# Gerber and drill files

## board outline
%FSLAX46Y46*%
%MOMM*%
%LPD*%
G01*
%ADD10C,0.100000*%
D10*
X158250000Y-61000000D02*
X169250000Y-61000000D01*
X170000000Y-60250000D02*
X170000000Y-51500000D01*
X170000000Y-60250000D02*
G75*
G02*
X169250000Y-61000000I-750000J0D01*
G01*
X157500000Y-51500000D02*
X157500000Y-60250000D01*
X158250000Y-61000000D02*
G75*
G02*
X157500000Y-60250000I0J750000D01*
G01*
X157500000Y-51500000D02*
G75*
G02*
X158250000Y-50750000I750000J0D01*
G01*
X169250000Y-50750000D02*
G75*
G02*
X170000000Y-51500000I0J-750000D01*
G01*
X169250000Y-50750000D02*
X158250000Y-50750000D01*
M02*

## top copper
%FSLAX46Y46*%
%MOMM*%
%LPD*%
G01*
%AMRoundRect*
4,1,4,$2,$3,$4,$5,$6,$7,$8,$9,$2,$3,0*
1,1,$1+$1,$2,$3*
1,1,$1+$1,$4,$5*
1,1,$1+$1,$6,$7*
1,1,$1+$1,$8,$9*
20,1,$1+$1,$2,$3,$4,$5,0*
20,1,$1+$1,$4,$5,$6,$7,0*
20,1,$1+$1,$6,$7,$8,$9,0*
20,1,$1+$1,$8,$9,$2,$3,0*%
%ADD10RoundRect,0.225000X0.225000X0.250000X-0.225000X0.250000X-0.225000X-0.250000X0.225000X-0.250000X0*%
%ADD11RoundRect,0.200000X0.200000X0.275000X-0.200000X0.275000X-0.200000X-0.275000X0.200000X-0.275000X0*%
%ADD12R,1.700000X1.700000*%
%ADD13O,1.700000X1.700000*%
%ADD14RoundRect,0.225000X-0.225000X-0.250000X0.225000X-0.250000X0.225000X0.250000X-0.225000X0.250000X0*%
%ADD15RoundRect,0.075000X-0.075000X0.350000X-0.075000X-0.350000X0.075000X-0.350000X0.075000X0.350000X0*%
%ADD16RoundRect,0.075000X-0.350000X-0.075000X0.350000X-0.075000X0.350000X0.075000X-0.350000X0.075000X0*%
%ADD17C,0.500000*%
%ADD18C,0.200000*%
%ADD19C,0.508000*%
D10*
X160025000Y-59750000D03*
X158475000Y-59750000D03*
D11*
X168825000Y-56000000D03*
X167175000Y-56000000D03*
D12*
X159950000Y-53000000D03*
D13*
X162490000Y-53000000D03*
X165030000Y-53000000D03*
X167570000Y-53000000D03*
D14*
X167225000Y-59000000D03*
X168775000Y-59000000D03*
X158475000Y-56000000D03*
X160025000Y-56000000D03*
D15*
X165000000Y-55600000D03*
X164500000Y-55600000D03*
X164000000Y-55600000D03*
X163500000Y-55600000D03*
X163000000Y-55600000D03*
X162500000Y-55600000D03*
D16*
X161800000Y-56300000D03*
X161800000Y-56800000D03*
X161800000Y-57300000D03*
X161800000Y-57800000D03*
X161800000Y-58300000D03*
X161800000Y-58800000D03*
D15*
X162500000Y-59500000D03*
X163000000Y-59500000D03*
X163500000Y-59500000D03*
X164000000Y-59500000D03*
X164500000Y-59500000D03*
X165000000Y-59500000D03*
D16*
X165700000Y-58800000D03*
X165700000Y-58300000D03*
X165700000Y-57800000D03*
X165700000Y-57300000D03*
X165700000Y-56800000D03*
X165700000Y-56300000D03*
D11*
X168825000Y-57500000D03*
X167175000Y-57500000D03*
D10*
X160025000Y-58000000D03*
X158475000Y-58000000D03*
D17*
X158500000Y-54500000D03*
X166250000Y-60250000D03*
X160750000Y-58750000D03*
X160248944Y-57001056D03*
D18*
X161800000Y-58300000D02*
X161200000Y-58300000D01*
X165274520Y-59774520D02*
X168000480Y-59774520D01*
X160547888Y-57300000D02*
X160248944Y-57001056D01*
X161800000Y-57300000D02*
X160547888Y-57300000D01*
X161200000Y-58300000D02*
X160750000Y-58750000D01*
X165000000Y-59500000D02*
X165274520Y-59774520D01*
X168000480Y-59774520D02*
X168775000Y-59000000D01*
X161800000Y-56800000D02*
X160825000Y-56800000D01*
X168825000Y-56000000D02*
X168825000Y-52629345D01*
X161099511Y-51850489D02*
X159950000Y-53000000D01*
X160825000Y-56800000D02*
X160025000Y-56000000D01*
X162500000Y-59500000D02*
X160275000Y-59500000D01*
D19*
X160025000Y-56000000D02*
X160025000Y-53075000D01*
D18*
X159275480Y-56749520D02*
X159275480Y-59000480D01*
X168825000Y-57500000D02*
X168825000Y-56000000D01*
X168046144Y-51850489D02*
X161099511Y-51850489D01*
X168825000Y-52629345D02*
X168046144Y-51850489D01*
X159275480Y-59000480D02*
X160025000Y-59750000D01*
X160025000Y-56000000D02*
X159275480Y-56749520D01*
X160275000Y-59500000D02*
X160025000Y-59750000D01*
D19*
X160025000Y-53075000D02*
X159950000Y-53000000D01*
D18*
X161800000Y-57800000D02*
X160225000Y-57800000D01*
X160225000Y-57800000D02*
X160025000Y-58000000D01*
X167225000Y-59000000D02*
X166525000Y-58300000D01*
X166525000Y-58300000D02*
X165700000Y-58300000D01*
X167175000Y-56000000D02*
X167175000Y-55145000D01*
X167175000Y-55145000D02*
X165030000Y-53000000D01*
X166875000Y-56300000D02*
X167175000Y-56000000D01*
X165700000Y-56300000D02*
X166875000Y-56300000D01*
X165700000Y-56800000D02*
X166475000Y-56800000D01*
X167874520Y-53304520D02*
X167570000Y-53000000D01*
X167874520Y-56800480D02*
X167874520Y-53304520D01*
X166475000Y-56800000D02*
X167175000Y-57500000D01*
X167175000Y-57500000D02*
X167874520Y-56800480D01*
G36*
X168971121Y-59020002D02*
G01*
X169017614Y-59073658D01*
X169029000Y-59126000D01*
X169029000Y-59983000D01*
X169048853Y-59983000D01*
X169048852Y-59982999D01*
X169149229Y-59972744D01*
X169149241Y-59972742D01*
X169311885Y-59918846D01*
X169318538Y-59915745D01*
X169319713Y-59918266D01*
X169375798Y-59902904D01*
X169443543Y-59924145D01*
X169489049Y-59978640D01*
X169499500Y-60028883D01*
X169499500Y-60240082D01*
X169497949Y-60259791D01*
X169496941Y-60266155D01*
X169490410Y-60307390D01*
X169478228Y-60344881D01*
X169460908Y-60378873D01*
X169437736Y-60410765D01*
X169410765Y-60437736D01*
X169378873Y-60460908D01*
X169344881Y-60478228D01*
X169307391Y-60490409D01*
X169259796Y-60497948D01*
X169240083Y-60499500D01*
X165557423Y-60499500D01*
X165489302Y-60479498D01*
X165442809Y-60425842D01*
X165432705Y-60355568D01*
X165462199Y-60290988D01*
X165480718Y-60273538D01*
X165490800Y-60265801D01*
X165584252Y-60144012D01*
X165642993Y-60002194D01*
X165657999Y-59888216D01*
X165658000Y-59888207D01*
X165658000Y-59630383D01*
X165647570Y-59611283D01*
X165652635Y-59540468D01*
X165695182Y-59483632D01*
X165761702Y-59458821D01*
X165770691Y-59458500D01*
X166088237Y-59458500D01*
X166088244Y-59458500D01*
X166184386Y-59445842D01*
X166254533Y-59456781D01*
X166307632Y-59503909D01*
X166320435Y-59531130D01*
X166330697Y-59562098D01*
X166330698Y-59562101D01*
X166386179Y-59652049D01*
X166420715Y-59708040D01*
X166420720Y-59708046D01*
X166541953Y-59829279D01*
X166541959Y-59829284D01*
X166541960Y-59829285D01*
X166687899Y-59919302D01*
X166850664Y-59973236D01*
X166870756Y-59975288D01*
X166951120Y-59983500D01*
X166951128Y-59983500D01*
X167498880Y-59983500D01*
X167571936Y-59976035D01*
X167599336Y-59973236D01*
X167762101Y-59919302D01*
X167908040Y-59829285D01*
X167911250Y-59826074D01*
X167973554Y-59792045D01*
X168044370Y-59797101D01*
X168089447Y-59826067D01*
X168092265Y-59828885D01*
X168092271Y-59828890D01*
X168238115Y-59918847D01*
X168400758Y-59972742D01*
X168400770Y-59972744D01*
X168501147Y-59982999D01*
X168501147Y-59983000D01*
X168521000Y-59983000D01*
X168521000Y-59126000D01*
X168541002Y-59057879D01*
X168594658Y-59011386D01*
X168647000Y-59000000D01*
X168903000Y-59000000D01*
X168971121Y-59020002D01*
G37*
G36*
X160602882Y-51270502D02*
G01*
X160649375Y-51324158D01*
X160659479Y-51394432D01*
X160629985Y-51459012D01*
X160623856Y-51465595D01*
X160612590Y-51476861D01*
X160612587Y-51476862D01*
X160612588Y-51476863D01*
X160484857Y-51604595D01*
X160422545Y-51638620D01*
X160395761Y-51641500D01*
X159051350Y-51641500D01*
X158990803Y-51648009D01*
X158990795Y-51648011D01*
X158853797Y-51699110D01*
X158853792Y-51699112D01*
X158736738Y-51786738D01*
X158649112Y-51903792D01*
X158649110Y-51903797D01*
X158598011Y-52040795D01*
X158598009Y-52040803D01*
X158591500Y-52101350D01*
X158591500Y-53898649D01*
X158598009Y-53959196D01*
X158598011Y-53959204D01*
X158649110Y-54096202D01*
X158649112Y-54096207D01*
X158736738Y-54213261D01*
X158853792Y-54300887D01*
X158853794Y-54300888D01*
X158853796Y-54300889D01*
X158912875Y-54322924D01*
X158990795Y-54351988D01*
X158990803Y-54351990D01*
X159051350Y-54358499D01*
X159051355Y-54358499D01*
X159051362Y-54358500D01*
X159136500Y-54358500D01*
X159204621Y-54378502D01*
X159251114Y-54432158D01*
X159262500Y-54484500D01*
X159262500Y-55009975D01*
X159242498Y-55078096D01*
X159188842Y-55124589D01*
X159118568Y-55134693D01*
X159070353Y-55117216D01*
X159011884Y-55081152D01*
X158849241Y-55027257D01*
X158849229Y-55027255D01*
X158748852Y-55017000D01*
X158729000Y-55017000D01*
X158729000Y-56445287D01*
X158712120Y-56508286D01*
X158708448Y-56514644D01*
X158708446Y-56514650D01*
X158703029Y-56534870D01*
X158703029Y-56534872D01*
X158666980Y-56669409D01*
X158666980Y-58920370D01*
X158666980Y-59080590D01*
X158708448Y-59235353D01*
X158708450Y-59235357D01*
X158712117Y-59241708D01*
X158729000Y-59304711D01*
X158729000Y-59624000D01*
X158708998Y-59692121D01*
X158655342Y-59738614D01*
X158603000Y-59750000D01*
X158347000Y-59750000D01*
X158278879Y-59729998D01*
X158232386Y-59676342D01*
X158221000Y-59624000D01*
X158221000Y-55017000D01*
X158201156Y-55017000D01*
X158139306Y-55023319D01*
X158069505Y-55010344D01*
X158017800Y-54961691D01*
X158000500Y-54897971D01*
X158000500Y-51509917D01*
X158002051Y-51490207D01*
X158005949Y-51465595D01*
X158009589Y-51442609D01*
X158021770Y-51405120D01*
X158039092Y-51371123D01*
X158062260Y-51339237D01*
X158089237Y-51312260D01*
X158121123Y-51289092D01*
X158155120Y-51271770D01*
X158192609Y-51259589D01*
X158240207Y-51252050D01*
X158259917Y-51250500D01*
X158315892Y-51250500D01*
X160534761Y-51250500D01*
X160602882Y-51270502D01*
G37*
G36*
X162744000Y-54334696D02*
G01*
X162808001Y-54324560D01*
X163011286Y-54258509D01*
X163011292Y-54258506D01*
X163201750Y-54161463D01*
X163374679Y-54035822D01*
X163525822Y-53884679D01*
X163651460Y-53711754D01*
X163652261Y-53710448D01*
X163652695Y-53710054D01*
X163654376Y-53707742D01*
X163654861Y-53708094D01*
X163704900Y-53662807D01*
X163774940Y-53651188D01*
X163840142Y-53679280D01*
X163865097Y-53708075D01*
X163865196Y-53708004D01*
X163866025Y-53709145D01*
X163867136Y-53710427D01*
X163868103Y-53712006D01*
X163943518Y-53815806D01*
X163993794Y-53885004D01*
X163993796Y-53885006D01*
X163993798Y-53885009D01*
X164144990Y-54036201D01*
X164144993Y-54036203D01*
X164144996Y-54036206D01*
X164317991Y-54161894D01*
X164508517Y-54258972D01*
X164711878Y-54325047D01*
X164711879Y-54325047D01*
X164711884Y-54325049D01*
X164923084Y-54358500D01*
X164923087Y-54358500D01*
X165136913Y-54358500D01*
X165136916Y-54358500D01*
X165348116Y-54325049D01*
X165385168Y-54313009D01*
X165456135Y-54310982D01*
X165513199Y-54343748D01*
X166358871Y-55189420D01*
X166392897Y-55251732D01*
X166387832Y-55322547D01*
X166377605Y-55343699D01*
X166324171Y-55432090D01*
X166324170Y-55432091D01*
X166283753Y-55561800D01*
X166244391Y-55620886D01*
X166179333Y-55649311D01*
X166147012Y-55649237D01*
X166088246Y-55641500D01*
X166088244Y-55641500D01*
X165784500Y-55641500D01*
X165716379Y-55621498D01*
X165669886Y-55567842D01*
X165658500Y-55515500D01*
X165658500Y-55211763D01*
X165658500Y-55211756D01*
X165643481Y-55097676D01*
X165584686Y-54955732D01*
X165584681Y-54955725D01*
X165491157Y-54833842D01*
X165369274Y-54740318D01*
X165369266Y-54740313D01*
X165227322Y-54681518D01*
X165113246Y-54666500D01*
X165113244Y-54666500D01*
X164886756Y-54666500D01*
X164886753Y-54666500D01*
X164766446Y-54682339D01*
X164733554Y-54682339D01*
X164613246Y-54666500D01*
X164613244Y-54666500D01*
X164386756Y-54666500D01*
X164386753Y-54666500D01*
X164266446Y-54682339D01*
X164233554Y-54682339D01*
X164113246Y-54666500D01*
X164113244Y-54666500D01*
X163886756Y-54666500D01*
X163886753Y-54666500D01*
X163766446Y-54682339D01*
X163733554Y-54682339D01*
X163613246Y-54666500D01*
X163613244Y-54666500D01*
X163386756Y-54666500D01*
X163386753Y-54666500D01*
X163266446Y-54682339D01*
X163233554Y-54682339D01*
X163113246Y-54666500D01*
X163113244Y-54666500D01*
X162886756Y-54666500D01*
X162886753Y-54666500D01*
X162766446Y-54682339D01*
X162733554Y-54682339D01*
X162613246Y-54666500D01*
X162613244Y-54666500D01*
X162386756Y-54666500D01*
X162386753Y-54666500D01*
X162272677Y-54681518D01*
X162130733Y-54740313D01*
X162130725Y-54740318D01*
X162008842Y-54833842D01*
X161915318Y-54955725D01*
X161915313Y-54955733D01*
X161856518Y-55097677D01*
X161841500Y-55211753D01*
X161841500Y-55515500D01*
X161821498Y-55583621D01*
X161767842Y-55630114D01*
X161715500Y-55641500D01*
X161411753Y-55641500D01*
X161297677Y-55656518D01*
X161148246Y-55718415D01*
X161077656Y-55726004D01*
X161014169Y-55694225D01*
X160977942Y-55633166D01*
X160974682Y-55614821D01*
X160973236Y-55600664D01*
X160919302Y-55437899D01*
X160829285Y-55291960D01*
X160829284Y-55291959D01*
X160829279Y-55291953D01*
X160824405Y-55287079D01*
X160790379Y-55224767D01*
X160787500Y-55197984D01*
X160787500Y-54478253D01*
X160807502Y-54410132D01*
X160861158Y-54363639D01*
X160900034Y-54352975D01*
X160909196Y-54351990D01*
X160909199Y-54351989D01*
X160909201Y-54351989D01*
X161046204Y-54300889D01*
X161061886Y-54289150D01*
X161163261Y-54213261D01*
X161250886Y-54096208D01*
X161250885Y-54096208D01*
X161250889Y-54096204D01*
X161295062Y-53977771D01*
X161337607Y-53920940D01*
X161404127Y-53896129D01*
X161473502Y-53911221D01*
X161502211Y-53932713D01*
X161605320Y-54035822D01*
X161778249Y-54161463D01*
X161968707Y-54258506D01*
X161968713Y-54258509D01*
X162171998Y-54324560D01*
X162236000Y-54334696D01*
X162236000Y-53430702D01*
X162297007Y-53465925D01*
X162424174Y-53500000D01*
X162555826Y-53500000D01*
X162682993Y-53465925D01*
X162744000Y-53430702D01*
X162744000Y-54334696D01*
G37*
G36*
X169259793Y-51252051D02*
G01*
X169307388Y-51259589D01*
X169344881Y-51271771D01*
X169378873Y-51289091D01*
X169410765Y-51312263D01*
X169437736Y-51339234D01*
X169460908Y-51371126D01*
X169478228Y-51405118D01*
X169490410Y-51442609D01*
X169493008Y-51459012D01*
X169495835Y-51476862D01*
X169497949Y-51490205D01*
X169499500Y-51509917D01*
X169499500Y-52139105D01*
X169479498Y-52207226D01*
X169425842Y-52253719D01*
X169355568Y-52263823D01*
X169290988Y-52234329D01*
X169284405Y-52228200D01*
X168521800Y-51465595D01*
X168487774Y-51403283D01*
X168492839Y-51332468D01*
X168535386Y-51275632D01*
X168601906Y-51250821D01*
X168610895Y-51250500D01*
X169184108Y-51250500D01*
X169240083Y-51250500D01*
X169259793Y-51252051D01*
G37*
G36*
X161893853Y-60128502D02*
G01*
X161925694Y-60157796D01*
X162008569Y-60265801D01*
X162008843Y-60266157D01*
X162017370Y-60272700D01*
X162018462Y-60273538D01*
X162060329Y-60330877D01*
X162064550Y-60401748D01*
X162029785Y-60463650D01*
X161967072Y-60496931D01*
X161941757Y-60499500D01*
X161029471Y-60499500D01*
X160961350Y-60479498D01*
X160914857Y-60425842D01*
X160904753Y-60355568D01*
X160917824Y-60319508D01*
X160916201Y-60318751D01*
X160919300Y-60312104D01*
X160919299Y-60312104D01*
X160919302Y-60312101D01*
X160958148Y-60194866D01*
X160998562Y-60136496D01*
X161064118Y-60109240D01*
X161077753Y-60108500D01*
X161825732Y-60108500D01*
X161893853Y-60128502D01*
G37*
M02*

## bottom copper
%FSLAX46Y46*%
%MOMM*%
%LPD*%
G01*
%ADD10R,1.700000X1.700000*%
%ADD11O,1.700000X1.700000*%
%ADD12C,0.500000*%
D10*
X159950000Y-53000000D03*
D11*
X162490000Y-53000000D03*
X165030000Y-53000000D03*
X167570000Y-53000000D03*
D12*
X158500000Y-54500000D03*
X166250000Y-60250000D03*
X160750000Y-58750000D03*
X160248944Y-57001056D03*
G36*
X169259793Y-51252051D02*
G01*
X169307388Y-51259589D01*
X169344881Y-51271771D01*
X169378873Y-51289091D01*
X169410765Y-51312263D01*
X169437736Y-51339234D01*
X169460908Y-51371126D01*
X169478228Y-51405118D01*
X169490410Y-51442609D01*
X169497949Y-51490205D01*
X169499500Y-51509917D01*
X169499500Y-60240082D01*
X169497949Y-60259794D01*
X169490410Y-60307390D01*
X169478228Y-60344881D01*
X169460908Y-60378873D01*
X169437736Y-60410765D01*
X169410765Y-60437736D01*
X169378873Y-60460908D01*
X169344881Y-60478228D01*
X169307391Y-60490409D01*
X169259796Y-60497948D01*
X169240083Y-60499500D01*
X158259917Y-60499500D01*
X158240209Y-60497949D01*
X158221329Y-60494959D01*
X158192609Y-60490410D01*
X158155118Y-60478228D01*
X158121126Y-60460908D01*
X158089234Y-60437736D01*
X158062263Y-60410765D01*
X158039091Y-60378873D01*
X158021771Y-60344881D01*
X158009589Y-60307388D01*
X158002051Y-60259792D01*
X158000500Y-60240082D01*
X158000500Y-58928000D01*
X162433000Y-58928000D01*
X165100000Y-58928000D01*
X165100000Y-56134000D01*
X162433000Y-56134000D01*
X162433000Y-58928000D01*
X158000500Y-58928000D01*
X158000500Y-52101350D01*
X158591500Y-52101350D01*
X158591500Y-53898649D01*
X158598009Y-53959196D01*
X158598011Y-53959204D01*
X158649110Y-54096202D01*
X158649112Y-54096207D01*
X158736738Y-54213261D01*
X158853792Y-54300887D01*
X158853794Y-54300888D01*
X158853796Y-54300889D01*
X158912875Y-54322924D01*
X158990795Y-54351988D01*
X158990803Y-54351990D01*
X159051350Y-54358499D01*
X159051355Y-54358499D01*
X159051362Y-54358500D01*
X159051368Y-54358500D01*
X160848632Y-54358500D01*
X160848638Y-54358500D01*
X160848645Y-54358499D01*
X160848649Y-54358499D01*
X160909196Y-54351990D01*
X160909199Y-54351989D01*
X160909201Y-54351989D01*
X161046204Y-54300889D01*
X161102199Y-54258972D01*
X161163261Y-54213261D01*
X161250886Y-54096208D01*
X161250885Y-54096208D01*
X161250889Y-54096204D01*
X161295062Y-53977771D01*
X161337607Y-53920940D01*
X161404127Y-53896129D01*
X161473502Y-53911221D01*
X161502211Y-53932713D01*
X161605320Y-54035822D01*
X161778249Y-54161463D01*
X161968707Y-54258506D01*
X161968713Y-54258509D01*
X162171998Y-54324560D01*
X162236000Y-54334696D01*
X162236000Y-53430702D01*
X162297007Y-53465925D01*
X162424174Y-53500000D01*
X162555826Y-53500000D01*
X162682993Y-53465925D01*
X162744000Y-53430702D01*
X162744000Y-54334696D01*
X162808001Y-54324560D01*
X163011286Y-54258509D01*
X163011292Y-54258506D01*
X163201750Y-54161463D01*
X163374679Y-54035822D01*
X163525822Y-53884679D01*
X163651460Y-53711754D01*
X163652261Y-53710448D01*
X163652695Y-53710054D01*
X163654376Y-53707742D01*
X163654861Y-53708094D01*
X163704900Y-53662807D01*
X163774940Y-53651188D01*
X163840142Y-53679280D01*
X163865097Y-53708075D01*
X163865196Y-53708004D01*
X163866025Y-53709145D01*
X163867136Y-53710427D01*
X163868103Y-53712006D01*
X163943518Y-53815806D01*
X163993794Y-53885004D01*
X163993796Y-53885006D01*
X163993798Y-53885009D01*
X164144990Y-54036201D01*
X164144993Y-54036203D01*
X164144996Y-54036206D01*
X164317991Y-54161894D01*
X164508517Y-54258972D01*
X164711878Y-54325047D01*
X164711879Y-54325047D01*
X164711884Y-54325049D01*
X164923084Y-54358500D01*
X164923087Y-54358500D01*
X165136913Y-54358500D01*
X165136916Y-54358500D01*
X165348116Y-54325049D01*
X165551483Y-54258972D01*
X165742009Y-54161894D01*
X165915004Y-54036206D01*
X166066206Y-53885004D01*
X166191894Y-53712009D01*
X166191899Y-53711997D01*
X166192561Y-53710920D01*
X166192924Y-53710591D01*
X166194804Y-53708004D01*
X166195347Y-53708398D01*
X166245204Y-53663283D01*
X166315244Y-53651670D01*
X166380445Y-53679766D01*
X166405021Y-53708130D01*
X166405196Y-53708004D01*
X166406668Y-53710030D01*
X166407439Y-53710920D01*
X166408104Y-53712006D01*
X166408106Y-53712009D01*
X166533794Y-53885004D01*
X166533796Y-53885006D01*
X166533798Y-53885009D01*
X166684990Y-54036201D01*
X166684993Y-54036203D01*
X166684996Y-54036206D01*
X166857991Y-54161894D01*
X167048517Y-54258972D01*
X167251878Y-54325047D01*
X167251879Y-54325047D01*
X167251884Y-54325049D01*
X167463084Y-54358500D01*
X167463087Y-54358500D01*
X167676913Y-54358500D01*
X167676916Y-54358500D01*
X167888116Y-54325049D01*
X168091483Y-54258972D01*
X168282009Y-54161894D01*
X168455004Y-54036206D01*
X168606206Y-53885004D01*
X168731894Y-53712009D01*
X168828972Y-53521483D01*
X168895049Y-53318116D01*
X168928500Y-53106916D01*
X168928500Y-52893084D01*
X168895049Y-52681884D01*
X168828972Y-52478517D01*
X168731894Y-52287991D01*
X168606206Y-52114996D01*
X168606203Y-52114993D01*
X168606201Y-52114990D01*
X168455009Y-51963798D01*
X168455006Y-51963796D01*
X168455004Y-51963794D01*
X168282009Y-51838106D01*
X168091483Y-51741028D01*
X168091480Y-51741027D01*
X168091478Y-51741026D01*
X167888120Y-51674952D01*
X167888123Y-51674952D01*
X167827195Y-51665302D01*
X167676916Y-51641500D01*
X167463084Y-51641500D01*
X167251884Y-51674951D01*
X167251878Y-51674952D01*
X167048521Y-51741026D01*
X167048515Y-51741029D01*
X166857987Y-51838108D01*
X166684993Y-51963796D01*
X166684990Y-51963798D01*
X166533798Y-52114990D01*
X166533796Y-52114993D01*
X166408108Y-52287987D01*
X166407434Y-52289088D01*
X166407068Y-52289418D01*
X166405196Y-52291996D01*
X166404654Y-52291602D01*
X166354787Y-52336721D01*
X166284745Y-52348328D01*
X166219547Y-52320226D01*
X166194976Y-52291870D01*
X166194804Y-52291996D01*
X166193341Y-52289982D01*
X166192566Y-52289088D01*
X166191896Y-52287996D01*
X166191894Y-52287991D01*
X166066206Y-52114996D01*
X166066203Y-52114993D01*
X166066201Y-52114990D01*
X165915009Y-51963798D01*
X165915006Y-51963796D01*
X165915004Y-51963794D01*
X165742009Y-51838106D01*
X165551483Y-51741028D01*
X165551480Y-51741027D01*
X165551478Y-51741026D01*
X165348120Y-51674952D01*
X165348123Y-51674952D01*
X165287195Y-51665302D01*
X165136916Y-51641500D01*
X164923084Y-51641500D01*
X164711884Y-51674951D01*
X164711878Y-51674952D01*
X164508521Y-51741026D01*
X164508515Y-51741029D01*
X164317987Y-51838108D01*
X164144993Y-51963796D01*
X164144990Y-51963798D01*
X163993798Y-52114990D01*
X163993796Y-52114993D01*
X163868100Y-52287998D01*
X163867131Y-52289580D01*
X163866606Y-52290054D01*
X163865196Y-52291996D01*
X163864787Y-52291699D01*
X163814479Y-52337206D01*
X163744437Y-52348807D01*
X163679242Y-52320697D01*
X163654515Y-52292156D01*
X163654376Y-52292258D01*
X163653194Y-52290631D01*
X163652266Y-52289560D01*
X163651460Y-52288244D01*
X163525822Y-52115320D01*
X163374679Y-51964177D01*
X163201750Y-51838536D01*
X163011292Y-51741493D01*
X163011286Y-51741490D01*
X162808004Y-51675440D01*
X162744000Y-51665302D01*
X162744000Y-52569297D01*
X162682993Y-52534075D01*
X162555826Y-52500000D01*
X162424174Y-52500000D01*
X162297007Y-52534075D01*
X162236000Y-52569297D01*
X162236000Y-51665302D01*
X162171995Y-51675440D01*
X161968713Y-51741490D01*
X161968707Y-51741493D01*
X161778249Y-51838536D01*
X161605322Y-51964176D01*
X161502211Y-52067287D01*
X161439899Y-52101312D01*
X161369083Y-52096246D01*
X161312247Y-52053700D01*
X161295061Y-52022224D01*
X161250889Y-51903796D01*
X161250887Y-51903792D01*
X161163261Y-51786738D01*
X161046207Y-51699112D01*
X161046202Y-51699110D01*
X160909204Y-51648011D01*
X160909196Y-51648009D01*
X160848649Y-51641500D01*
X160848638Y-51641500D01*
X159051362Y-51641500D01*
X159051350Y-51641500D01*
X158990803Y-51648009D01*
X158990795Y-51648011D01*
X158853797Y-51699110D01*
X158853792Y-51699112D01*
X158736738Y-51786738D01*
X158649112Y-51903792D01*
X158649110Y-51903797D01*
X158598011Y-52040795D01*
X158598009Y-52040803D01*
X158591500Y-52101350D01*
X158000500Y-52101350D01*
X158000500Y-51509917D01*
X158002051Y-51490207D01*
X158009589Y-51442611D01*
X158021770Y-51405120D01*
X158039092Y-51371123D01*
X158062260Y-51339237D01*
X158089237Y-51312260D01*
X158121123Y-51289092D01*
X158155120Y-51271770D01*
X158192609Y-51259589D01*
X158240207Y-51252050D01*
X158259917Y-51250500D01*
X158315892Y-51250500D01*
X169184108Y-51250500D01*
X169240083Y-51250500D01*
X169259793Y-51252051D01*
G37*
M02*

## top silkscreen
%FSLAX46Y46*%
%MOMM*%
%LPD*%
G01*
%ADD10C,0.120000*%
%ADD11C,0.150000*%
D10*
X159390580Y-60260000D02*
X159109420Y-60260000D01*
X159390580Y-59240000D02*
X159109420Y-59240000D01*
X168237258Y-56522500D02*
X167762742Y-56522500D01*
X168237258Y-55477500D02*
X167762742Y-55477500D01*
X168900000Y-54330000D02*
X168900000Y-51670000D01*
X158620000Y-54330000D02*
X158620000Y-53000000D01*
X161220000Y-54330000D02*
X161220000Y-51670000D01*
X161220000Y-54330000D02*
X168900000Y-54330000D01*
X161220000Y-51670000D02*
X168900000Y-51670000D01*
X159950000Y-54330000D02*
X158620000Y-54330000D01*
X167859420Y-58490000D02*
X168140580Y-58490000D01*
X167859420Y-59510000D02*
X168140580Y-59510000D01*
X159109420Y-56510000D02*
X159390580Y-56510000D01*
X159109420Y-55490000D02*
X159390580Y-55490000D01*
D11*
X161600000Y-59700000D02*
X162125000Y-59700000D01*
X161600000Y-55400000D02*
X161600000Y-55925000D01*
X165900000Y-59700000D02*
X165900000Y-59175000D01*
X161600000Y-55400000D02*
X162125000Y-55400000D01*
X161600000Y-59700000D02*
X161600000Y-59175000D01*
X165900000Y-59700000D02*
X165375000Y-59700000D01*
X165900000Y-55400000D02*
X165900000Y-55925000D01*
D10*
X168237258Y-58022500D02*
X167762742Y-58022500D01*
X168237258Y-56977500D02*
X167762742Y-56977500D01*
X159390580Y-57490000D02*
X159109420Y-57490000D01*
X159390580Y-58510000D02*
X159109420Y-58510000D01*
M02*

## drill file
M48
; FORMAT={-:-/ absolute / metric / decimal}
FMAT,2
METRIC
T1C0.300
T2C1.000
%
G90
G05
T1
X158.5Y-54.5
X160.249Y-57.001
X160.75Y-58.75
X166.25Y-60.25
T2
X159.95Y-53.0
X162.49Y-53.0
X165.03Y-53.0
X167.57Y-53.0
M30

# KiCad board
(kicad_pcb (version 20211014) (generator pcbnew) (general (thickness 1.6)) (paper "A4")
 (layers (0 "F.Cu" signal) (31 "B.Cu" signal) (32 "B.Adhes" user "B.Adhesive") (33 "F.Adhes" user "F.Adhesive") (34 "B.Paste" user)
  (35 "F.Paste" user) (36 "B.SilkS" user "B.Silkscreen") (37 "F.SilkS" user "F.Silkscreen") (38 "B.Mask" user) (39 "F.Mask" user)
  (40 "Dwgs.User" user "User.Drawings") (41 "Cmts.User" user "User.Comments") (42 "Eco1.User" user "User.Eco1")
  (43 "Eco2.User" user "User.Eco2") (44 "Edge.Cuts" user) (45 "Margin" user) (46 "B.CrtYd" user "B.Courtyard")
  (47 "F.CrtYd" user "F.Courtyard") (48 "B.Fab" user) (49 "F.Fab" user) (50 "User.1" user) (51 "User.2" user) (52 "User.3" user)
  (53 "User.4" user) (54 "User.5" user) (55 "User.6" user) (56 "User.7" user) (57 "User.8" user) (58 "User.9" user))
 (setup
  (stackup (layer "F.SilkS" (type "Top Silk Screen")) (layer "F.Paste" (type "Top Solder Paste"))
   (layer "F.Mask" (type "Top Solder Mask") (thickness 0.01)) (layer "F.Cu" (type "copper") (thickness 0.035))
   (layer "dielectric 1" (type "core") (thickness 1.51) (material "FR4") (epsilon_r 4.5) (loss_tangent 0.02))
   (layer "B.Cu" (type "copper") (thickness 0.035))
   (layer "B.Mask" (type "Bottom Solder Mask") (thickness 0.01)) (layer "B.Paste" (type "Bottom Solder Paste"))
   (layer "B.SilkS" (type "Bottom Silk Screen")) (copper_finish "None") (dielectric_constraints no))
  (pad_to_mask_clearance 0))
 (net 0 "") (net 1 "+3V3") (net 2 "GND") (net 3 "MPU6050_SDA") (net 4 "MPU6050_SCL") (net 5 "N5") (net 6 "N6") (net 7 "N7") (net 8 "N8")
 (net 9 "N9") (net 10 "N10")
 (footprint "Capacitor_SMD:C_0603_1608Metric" (layer "F.Cu") (at 159.25 59.75 180)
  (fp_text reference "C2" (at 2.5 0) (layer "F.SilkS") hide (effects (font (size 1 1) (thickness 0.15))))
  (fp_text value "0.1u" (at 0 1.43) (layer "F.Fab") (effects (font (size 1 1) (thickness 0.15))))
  (fp_line (start -0.14058 -0.51) (end 0.14058 -0.51) (layer "F.SilkS") (width 0.12))
  (fp_line (start -0.14058 0.51) (end 0.14058 0.51) (layer "F.SilkS") (width 0.12))
  (pad "1" smd roundrect (at -0.775 0 180) (size 0.9 0.95) (layers "F.Cu" "F.Paste" "F.Mask") (roundrect_rratio 0.25) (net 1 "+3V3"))
  (pad "2" smd roundrect (at 0.775 0 180) (size 0.9 0.95) (layers "F.Cu" "F.Paste" "F.Mask") (roundrect_rratio 0.25) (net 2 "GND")))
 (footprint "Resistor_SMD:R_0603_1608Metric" (layer "F.Cu") (at 168 56 180)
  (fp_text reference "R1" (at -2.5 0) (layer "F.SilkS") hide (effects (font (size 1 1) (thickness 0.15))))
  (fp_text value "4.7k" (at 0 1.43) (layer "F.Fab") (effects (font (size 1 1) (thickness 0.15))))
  (fp_line (start -0.237258 -0.5225) (end 0.237258 -0.5225) (layer "F.SilkS") (width 0.12))
  (fp_line (start -0.237258 0.5225) (end 0.237258 0.5225) (layer "F.SilkS") (width 0.12))
  (pad "1" smd roundrect (at -0.825 0 180) (size 0.8 0.95) (layers "F.Cu" "F.Paste" "F.Mask") (roundrect_rratio 0.25) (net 1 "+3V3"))
  (pad "2" smd roundrect (at 0.825 0 180) (size 0.8 0.95) (layers "F.Cu" "F.Paste" "F.Mask") (roundrect_rratio 0.25) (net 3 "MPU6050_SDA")))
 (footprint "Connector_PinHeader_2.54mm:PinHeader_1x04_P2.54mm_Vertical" (layer "F.Cu") (at 159.95 53 90)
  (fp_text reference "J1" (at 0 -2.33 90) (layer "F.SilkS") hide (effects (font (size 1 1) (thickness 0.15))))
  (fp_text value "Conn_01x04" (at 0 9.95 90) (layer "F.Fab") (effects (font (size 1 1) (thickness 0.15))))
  (fp_line (start -1.33 8.95) (end 1.33 8.95) (layer "F.SilkS") (width 0.12))
  (fp_line (start -1.33 -1.33) (end 0 -1.33) (layer "F.SilkS") (width 0.12))
  (fp_line (start -1.33 1.27) (end 1.33 1.27) (layer "F.SilkS") (width 0.12))
  (fp_line (start -1.33 1.27) (end -1.33 8.95) (layer "F.SilkS") (width 0.12))
  (fp_line (start 1.33 1.27) (end 1.33 8.95) (layer "F.SilkS") (width 0.12))
  (fp_line (start -1.33 0) (end -1.33 -1.33) (layer "F.SilkS") (width 0.12))
  (pad "1" thru_hole rect (at 0 0 90) (size 1.7 1.7) (drill 1) (layers *.Cu *.Mask) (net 1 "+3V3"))
  (pad "2" thru_hole oval (at 0 2.54 90) (size 1.7 1.7) (drill 1) (layers *.Cu *.Mask) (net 2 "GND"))
  (pad "3" thru_hole oval (at 0 5.08 90) (size 1.7 1.7) (drill 1) (layers *.Cu *.Mask) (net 3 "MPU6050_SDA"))
  (pad "4" thru_hole oval (at 0 7.62 90) (size 1.7 1.7) (drill 1) (layers *.Cu *.Mask) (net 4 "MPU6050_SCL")))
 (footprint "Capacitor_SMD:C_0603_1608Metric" (layer "F.Cu") (at 168 59)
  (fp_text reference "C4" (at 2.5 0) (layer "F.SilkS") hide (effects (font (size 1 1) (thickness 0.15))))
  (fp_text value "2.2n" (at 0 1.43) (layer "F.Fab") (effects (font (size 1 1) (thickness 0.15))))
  (fp_line (start -0.14058 -0.51) (end 0.14058 -0.51) (layer "F.SilkS") (width 0.12))
  (fp_line (start -0.14058 0.51) (end 0.14058 0.51) (layer "F.SilkS") (width 0.12))
  (pad "1" smd roundrect (at -0.775 0) (size 0.9 0.95) (layers "F.Cu" "F.Paste" "F.Mask") (roundrect_rratio 0.25) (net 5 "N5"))
  (pad "2" smd roundrect (at 0.775 0) (size 0.9 0.95) (layers "F.Cu" "F.Paste" "F.Mask") (roundrect_rratio 0.25) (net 2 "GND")))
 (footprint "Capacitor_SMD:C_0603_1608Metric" (layer "F.Cu") (at 159.25 56)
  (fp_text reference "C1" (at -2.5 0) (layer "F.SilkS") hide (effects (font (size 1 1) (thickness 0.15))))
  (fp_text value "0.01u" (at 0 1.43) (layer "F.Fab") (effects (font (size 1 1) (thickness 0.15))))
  (fp_line (start -0.14058 0.51) (end 0.14058 0.51) (layer "F.SilkS") (width 0.12))
  (fp_line (start -0.14058 -0.51) (end 0.14058 -0.51) (layer "F.SilkS") (width 0.12))
  (pad "1" smd roundrect (at -0.775 0) (size 0.9 0.95) (layers "F.Cu" "F.Paste" "F.Mask") (roundrect_rratio 0.25) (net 2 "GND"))
  (pad "2" smd roundrect (at 0.775 0) (size 0.9 0.95) (layers "F.Cu" "F.Paste" "F.Mask") (roundrect_rratio 0.25) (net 1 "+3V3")))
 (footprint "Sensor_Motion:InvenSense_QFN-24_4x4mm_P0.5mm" (layer "F.Cu") (at 163.75 57.55 -90)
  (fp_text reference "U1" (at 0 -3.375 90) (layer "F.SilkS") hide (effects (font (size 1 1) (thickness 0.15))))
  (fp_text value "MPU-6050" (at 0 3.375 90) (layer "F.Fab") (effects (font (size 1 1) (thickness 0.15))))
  (fp_line (start 2.15 2.15) (end 2.15 1.625) (layer "F.SilkS") (width 0.15))
  (fp_line (start -2.15 2.15) (end -1.625 2.15) (layer "F.SilkS") (width 0.15))
  (fp_line (start 2.15 -2.15) (end 1.625 -2.15) (layer "F.SilkS") (width 0.15))
  (fp_line (start -2.15 2.15) (end -2.15 1.625) (layer "F.SilkS") (width 0.15))
  (fp_line (start 2.15 2.15) (end 1.625 2.15) (layer "F.SilkS") (width 0.15))
  (fp_line (start 2.15 -2.15) (end 2.15 -1.625) (layer "F.SilkS") (width 0.15))
  (fp_line (start -2.15 -2.15) (end -1.625 -2.15) (layer "F.SilkS") (width 0.15))
  (pad "1" smd roundrect (at -1.95 -1.25 270) (size 0.85 0.3) (layers "F.Cu" "F.Paste" "F.Mask") (roundrect_rratio 0.25) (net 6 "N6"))
  (pad "2" smd roundrect (at -1.95 -0.75 270) (size 0.85 0.3) (layers "F.Cu" "F.Paste" "F.Mask") (roundrect_rratio 0.25))
  (pad "3" smd roundrect (at -1.95 -0.25 270) (size 0.85 0.3) (layers "F.Cu" "F.Paste" "F.Mask") (roundrect_rratio 0.25))
  (pad "4" smd roundrect (at -1.95 0.25 270) (size 0.85 0.3) (layers "F.Cu" "F.Paste" "F.Mask") (roundrect_rratio 0.25))
  (pad "5" smd roundrect (at -1.95 0.75 270) (size 0.85 0.3) (layers "F.Cu" "F.Paste" "F.Mask") (roundrect_rratio 0.25))
  (pad "6" smd roundrect (at -1.95 1.25 270) (size 0.85 0.3) (layers "F.Cu" "F.Paste" "F.Mask") (roundrect_rratio 0.25) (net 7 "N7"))
  (pad "7" smd roundrect (at -1.25 1.95) (size 0.85 0.3) (layers "F.Cu" "F.Paste" "F.Mask") (roundrect_rratio 0.25) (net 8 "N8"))
  (pad "8" smd roundrect (at -0.75 1.95) (size 0.85 0.3) (layers "F.Cu" "F.Paste" "F.Mask") (roundrect_rratio 0.25) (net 1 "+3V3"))
  (pad "9" smd roundrect (at -0.25 1.95) (size 0.85 0.3) (layers "F.Cu" "F.Paste" "F.Mask") (roundrect_rratio 0.25) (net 2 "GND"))
  (pad "10" smd roundrect (at 0.25 1.95) (size 0.85 0.3) (layers "F.Cu" "F.Paste" "F.Mask") (roundrect_rratio 0.25) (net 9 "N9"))
  (pad "11" smd roundrect (at 0.75 1.95) (size 0.85 0.3) (layers "F.Cu" "F.Paste" "F.Mask") (roundrect_rratio 0.25) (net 2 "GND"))
  (pad "12" smd roundrect (at 1.25 1.95) (size 0.85 0.3) (layers "F.Cu" "F.Paste" "F.Mask") (roundrect_rratio 0.25) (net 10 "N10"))
  (pad "13" smd roundrect (at 1.95 1.25 270) (size 0.85 0.3) (layers "F.Cu" "F.Paste" "F.Mask") (roundrect_rratio 0.25) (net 1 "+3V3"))
  (pad "14" smd roundrect (at 1.95 0.75 270) (size 0.85 0.3) (layers "F.Cu" "F.Paste" "F.Mask") (roundrect_rratio 0.25))
  (pad "15" smd roundrect (at 1.95 0.25 270) (size 0.85 0.3) (layers "F.Cu" "F.Paste" "F.Mask") (roundrect_rratio 0.25))
  (pad "16" smd roundrect (at 1.95 -0.25 270) (size 0.85 0.3) (layers "F.Cu" "F.Paste" "F.Mask") (roundrect_rratio 0.25))
  (pad "17" smd roundrect (at 1.95 -0.75 270) (size 0.85 0.3) (layers "F.Cu" "F.Paste" "F.Mask") (roundrect_rratio 0.25))
  (pad "18" smd roundrect (at 1.95 -1.25 270) (size 0.85 0.3) (layers "F.Cu" "F.Paste" "F.Mask") (roundrect_rratio 0.25) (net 2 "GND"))
  (pad "19" smd roundrect (at 1.25 -1.95) (size 0.85 0.3) (layers "F.Cu" "F.Paste" "F.Mask") (roundrect_rratio 0.25))
  (pad "20" smd roundrect (at 0.75 -1.95) (size 0.85 0.3) (layers "F.Cu" "F.Paste" "F.Mask") (roundrect_rratio 0.25) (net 5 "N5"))
  (pad "21" smd roundrect (at 0.25 -1.95) (size 0.85 0.3) (layers "F.Cu" "F.Paste" "F.Mask") (roundrect_rratio 0.25))
  (pad "22" smd roundrect (at -0.25 -1.95) (size 0.85 0.3) (layers "F.Cu" "F.Paste" "F.Mask") (roundrect_rratio 0.25))
  (pad "23" smd roundrect (at -0.75 -1.95) (size 0.85 0.3) (layers "F.Cu" "F.Paste" "F.Mask") (roundrect_rratio 0.25) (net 4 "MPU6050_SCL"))
  (pad "24" smd roundrect (at -1.25 -1.95) (size 0.85 0.3) (layers "F.Cu" "F.Paste" "F.Mask") (roundrect_rratio 0.25) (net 3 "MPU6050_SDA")))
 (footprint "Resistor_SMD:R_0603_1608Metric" (layer "F.Cu") (at 168 57.5 180)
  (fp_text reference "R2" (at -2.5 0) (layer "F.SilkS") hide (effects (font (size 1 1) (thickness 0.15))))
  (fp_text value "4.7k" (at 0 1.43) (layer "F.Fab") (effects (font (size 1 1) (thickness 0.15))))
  (fp_line (start -0.237258 -0.5225) (end 0.237258 -0.5225) (layer "F.SilkS") (width 0.12))
  (fp_line (start -0.237258 0.5225) (end 0.237258 0.5225) (layer "F.SilkS") (width 0.12))
  (pad "1" smd roundrect (at -0.825 0 180) (size 0.8 0.95) (layers "F.Cu" "F.Paste" "F.Mask") (roundrect_rratio 0.25) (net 1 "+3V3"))
  (pad "2" smd roundrect (at 0.825 0 180) (size 0.8 0.95) (layers "F.Cu" "F.Paste" "F.Mask") (roundrect_rratio 0.25) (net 4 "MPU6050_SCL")))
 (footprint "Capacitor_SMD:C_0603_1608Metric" (layer "F.Cu") (at 159.25 58 180)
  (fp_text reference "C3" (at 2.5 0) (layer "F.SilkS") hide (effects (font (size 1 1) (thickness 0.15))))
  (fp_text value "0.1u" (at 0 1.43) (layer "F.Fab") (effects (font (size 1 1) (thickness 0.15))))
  (fp_line (start -0.14058 0.51) (end 0.14058 0.51) (layer "F.SilkS") (width 0.12))
  (fp_line (start -0.14058 -0.51) (end 0.14058 -0.51) (layer "F.SilkS") (width 0.12))
  (pad "1" smd roundrect (at -0.775 0 180) (size 0.9 0.95) (layers "F.Cu" "F.Paste" "F.Mask") (roundrect_rratio 0.25) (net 9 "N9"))
  (pad "2" smd roundrect (at 0.775 0 180) (size 0.9 0.95) (layers "F.Cu" "F.Paste" "F.Mask") (roundrect_rratio 0.25) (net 2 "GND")))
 (gr_line (start 158.25 61) (end 169.25 61) (layer "Edge.Cuts") (width 0.1))
 (gr_line (start 170 60.25) (end 170 51.5) (layer "Edge.Cuts") (width 0.1))
 (gr_arc (start 170 60.25) (mid 169.78033 60.78033) (end 169.25 61) (layer "Edge.Cuts") (width 0.1))
 (gr_line (start 157.5 51.5) (end 157.5 60.25) (layer "Edge.Cuts") (width 0.1))
 (gr_arc (start 158.25 61) (mid 157.71967 60.78033) (end 157.5 60.25) (layer "Edge.Cuts") (width 0.1))
 (gr_arc (start 157.5 51.5) (mid 157.71967 50.96967) (end 158.25 50.75) (layer "Edge.Cuts") (width 0.1))
 (gr_arc (start 169.25 50.75) (mid 169.78033 50.96967) (end 170 51.5) (layer "Edge.Cuts") (width 0.1))
 (gr_line (start 169.25 50.75) (end 158.25 50.75) (layer "Edge.Cuts") (width 0.1))
 (segment (start 161.8 58.3) (end 161.2 58.3) (width 0.2) (layer "F.Cu") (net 2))
 (segment (start 165.27452 59.77452) (end 168.00048 59.77452) (width 0.2) (layer "F.Cu") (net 2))
 (segment (start 160.547888 57.3) (end 160.248944 57.001056) (width 0.2) (layer "F.Cu") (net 2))
 (segment (start 161.8 57.3) (end 160.547888 57.3) (width 0.2) (layer "F.Cu") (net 2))
 (segment (start 161.2 58.3) (end 160.75 58.75) (width 0.2) (layer "F.Cu") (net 2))
 (segment (start 165 59.5) (end 165.27452 59.77452) (width 0.2) (layer "F.Cu") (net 2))
 (segment (start 168.00048 59.77452) (end 168.775 59) (width 0.2) (layer "F.Cu") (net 2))
 (via (at 158.5 54.5) (size 0.5) (drill 0.3) (layers "F.Cu" "B.Cu") (free) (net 2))
 (via (at 166.25 60.25) (size 0.5) (drill 0.3) (layers "F.Cu" "B.Cu") (free) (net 2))
 (via (at 160.75 58.75) (size 0.5) (drill 0.3) (layers "F.Cu" "B.Cu") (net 2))
 (via (at 160.248944 57.001056) (size 0.5) (drill 0.3) (layers "F.Cu" "B.Cu") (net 2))
 (segment (start 161.8 56.8) (end 160.825 56.8) (width 0.2) (layer "F.Cu") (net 1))
 (segment (start 168.825 56) (end 168.825 52.629345) (width 0.2) (layer "F.Cu") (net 1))
 (segment (start 161.099511 51.850489) (end 159.95 53) (width 0.2) (layer "F.Cu") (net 1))
 (segment (start 160.825 56.8) (end 160.025 56) (width 0.2) (layer "F.Cu") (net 1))
 (segment (start 162.5 59.5) (end 160.275 59.5) (width 0.2) (layer "F.Cu") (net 1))
 (segment (start 160.025 56) (end 160.025 53.075) (width 0.508) (layer "F.Cu") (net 1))
 (segment (start 159.27548 56.74952) (end 159.27548 59.00048) (width 0.2) (layer "F.Cu") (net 1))
 (segment (start 168.825 57.5) (end 168.825 56) (width 0.2) (layer "F.Cu") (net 1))
 (segment (start 168.046144 51.850489) (end 161.099511 51.850489) (width 0.2) (layer "F.Cu") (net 1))
 (segment (start 168.825 52.629345) (end 168.046144 51.850489) (width 0.2) (layer "F.Cu") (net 1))
 (segment (start 159.27548 59.00048) (end 160.025 59.75) (width 0.2) (layer "F.Cu") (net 1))
 (segment (start 160.025 56) (end 159.27548 56.74952) (width 0.2) (layer "F.Cu") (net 1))
 (segment (start 160.275 59.5) (end 160.025 59.75) (width 0.2) (layer "F.Cu") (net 1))
 (segment (start 160.025 53.075) (end 159.95 53) (width 0.508) (layer "F.Cu") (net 1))
 (segment (start 161.8 57.8) (end 160.225 57.8) (width 0.2) (layer "F.Cu") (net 9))
 (segment (start 160.225 57.8) (end 160.025 58) (width 0.2) (layer "F.Cu") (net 9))
 (segment (start 167.225 59) (end 166.525 58.3) (width 0.2) (layer "F.Cu") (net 5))
 (segment (start 166.525 58.3) (end 165.7 58.3) (width 0.2) (layer "F.Cu") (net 5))
 (segment (start 167.175 56) (end 167.175 55.145) (width 0.2) (layer "F.Cu") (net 3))
 (segment (start 167.175 55.145) (end 165.03 53) (width 0.2) (layer "F.Cu") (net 3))
 (segment (start 166.875 56.3) (end 167.175 56) (width 0.2) (layer "F.Cu") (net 3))
 (segment (start 165.7 56.3) (end 166.875 56.3) (width 0.2) (layer "F.Cu") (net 3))
 (segment (start 165.7 56.8) (end 166.475 56.8) (width 0.2) (layer "F.Cu") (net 4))
 (segment (start 167.87452 53.30452) (end 167.57 53) (width 0.2) (layer "F.Cu") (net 4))
 (segment (start 167.87452 56.80048) (end 167.87452 53.30452) (width 0.2) (layer "F.Cu") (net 4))
 (segment (start 166.475 56.8) (end 167.175 57.5) (width 0.2) (layer "F.Cu") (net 4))
 (segment (start 167.175 57.5) (end 167.87452 56.80048) (width 0.2) (layer "F.Cu") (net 4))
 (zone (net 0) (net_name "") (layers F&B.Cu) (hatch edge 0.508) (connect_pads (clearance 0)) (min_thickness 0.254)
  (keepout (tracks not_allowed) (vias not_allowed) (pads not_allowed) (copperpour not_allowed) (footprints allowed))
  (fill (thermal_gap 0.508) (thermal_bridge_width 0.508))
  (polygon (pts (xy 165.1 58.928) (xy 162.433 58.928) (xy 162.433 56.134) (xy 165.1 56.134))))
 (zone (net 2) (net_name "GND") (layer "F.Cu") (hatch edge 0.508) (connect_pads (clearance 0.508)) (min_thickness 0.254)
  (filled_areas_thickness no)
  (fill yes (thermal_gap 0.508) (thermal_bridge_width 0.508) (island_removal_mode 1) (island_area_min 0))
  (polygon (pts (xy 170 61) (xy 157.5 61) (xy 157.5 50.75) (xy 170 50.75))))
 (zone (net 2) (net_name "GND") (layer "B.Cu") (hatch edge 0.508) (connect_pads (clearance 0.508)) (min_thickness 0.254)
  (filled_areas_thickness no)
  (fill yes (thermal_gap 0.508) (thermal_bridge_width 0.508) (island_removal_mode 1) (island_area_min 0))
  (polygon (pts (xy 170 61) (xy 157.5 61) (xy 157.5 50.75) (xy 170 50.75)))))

